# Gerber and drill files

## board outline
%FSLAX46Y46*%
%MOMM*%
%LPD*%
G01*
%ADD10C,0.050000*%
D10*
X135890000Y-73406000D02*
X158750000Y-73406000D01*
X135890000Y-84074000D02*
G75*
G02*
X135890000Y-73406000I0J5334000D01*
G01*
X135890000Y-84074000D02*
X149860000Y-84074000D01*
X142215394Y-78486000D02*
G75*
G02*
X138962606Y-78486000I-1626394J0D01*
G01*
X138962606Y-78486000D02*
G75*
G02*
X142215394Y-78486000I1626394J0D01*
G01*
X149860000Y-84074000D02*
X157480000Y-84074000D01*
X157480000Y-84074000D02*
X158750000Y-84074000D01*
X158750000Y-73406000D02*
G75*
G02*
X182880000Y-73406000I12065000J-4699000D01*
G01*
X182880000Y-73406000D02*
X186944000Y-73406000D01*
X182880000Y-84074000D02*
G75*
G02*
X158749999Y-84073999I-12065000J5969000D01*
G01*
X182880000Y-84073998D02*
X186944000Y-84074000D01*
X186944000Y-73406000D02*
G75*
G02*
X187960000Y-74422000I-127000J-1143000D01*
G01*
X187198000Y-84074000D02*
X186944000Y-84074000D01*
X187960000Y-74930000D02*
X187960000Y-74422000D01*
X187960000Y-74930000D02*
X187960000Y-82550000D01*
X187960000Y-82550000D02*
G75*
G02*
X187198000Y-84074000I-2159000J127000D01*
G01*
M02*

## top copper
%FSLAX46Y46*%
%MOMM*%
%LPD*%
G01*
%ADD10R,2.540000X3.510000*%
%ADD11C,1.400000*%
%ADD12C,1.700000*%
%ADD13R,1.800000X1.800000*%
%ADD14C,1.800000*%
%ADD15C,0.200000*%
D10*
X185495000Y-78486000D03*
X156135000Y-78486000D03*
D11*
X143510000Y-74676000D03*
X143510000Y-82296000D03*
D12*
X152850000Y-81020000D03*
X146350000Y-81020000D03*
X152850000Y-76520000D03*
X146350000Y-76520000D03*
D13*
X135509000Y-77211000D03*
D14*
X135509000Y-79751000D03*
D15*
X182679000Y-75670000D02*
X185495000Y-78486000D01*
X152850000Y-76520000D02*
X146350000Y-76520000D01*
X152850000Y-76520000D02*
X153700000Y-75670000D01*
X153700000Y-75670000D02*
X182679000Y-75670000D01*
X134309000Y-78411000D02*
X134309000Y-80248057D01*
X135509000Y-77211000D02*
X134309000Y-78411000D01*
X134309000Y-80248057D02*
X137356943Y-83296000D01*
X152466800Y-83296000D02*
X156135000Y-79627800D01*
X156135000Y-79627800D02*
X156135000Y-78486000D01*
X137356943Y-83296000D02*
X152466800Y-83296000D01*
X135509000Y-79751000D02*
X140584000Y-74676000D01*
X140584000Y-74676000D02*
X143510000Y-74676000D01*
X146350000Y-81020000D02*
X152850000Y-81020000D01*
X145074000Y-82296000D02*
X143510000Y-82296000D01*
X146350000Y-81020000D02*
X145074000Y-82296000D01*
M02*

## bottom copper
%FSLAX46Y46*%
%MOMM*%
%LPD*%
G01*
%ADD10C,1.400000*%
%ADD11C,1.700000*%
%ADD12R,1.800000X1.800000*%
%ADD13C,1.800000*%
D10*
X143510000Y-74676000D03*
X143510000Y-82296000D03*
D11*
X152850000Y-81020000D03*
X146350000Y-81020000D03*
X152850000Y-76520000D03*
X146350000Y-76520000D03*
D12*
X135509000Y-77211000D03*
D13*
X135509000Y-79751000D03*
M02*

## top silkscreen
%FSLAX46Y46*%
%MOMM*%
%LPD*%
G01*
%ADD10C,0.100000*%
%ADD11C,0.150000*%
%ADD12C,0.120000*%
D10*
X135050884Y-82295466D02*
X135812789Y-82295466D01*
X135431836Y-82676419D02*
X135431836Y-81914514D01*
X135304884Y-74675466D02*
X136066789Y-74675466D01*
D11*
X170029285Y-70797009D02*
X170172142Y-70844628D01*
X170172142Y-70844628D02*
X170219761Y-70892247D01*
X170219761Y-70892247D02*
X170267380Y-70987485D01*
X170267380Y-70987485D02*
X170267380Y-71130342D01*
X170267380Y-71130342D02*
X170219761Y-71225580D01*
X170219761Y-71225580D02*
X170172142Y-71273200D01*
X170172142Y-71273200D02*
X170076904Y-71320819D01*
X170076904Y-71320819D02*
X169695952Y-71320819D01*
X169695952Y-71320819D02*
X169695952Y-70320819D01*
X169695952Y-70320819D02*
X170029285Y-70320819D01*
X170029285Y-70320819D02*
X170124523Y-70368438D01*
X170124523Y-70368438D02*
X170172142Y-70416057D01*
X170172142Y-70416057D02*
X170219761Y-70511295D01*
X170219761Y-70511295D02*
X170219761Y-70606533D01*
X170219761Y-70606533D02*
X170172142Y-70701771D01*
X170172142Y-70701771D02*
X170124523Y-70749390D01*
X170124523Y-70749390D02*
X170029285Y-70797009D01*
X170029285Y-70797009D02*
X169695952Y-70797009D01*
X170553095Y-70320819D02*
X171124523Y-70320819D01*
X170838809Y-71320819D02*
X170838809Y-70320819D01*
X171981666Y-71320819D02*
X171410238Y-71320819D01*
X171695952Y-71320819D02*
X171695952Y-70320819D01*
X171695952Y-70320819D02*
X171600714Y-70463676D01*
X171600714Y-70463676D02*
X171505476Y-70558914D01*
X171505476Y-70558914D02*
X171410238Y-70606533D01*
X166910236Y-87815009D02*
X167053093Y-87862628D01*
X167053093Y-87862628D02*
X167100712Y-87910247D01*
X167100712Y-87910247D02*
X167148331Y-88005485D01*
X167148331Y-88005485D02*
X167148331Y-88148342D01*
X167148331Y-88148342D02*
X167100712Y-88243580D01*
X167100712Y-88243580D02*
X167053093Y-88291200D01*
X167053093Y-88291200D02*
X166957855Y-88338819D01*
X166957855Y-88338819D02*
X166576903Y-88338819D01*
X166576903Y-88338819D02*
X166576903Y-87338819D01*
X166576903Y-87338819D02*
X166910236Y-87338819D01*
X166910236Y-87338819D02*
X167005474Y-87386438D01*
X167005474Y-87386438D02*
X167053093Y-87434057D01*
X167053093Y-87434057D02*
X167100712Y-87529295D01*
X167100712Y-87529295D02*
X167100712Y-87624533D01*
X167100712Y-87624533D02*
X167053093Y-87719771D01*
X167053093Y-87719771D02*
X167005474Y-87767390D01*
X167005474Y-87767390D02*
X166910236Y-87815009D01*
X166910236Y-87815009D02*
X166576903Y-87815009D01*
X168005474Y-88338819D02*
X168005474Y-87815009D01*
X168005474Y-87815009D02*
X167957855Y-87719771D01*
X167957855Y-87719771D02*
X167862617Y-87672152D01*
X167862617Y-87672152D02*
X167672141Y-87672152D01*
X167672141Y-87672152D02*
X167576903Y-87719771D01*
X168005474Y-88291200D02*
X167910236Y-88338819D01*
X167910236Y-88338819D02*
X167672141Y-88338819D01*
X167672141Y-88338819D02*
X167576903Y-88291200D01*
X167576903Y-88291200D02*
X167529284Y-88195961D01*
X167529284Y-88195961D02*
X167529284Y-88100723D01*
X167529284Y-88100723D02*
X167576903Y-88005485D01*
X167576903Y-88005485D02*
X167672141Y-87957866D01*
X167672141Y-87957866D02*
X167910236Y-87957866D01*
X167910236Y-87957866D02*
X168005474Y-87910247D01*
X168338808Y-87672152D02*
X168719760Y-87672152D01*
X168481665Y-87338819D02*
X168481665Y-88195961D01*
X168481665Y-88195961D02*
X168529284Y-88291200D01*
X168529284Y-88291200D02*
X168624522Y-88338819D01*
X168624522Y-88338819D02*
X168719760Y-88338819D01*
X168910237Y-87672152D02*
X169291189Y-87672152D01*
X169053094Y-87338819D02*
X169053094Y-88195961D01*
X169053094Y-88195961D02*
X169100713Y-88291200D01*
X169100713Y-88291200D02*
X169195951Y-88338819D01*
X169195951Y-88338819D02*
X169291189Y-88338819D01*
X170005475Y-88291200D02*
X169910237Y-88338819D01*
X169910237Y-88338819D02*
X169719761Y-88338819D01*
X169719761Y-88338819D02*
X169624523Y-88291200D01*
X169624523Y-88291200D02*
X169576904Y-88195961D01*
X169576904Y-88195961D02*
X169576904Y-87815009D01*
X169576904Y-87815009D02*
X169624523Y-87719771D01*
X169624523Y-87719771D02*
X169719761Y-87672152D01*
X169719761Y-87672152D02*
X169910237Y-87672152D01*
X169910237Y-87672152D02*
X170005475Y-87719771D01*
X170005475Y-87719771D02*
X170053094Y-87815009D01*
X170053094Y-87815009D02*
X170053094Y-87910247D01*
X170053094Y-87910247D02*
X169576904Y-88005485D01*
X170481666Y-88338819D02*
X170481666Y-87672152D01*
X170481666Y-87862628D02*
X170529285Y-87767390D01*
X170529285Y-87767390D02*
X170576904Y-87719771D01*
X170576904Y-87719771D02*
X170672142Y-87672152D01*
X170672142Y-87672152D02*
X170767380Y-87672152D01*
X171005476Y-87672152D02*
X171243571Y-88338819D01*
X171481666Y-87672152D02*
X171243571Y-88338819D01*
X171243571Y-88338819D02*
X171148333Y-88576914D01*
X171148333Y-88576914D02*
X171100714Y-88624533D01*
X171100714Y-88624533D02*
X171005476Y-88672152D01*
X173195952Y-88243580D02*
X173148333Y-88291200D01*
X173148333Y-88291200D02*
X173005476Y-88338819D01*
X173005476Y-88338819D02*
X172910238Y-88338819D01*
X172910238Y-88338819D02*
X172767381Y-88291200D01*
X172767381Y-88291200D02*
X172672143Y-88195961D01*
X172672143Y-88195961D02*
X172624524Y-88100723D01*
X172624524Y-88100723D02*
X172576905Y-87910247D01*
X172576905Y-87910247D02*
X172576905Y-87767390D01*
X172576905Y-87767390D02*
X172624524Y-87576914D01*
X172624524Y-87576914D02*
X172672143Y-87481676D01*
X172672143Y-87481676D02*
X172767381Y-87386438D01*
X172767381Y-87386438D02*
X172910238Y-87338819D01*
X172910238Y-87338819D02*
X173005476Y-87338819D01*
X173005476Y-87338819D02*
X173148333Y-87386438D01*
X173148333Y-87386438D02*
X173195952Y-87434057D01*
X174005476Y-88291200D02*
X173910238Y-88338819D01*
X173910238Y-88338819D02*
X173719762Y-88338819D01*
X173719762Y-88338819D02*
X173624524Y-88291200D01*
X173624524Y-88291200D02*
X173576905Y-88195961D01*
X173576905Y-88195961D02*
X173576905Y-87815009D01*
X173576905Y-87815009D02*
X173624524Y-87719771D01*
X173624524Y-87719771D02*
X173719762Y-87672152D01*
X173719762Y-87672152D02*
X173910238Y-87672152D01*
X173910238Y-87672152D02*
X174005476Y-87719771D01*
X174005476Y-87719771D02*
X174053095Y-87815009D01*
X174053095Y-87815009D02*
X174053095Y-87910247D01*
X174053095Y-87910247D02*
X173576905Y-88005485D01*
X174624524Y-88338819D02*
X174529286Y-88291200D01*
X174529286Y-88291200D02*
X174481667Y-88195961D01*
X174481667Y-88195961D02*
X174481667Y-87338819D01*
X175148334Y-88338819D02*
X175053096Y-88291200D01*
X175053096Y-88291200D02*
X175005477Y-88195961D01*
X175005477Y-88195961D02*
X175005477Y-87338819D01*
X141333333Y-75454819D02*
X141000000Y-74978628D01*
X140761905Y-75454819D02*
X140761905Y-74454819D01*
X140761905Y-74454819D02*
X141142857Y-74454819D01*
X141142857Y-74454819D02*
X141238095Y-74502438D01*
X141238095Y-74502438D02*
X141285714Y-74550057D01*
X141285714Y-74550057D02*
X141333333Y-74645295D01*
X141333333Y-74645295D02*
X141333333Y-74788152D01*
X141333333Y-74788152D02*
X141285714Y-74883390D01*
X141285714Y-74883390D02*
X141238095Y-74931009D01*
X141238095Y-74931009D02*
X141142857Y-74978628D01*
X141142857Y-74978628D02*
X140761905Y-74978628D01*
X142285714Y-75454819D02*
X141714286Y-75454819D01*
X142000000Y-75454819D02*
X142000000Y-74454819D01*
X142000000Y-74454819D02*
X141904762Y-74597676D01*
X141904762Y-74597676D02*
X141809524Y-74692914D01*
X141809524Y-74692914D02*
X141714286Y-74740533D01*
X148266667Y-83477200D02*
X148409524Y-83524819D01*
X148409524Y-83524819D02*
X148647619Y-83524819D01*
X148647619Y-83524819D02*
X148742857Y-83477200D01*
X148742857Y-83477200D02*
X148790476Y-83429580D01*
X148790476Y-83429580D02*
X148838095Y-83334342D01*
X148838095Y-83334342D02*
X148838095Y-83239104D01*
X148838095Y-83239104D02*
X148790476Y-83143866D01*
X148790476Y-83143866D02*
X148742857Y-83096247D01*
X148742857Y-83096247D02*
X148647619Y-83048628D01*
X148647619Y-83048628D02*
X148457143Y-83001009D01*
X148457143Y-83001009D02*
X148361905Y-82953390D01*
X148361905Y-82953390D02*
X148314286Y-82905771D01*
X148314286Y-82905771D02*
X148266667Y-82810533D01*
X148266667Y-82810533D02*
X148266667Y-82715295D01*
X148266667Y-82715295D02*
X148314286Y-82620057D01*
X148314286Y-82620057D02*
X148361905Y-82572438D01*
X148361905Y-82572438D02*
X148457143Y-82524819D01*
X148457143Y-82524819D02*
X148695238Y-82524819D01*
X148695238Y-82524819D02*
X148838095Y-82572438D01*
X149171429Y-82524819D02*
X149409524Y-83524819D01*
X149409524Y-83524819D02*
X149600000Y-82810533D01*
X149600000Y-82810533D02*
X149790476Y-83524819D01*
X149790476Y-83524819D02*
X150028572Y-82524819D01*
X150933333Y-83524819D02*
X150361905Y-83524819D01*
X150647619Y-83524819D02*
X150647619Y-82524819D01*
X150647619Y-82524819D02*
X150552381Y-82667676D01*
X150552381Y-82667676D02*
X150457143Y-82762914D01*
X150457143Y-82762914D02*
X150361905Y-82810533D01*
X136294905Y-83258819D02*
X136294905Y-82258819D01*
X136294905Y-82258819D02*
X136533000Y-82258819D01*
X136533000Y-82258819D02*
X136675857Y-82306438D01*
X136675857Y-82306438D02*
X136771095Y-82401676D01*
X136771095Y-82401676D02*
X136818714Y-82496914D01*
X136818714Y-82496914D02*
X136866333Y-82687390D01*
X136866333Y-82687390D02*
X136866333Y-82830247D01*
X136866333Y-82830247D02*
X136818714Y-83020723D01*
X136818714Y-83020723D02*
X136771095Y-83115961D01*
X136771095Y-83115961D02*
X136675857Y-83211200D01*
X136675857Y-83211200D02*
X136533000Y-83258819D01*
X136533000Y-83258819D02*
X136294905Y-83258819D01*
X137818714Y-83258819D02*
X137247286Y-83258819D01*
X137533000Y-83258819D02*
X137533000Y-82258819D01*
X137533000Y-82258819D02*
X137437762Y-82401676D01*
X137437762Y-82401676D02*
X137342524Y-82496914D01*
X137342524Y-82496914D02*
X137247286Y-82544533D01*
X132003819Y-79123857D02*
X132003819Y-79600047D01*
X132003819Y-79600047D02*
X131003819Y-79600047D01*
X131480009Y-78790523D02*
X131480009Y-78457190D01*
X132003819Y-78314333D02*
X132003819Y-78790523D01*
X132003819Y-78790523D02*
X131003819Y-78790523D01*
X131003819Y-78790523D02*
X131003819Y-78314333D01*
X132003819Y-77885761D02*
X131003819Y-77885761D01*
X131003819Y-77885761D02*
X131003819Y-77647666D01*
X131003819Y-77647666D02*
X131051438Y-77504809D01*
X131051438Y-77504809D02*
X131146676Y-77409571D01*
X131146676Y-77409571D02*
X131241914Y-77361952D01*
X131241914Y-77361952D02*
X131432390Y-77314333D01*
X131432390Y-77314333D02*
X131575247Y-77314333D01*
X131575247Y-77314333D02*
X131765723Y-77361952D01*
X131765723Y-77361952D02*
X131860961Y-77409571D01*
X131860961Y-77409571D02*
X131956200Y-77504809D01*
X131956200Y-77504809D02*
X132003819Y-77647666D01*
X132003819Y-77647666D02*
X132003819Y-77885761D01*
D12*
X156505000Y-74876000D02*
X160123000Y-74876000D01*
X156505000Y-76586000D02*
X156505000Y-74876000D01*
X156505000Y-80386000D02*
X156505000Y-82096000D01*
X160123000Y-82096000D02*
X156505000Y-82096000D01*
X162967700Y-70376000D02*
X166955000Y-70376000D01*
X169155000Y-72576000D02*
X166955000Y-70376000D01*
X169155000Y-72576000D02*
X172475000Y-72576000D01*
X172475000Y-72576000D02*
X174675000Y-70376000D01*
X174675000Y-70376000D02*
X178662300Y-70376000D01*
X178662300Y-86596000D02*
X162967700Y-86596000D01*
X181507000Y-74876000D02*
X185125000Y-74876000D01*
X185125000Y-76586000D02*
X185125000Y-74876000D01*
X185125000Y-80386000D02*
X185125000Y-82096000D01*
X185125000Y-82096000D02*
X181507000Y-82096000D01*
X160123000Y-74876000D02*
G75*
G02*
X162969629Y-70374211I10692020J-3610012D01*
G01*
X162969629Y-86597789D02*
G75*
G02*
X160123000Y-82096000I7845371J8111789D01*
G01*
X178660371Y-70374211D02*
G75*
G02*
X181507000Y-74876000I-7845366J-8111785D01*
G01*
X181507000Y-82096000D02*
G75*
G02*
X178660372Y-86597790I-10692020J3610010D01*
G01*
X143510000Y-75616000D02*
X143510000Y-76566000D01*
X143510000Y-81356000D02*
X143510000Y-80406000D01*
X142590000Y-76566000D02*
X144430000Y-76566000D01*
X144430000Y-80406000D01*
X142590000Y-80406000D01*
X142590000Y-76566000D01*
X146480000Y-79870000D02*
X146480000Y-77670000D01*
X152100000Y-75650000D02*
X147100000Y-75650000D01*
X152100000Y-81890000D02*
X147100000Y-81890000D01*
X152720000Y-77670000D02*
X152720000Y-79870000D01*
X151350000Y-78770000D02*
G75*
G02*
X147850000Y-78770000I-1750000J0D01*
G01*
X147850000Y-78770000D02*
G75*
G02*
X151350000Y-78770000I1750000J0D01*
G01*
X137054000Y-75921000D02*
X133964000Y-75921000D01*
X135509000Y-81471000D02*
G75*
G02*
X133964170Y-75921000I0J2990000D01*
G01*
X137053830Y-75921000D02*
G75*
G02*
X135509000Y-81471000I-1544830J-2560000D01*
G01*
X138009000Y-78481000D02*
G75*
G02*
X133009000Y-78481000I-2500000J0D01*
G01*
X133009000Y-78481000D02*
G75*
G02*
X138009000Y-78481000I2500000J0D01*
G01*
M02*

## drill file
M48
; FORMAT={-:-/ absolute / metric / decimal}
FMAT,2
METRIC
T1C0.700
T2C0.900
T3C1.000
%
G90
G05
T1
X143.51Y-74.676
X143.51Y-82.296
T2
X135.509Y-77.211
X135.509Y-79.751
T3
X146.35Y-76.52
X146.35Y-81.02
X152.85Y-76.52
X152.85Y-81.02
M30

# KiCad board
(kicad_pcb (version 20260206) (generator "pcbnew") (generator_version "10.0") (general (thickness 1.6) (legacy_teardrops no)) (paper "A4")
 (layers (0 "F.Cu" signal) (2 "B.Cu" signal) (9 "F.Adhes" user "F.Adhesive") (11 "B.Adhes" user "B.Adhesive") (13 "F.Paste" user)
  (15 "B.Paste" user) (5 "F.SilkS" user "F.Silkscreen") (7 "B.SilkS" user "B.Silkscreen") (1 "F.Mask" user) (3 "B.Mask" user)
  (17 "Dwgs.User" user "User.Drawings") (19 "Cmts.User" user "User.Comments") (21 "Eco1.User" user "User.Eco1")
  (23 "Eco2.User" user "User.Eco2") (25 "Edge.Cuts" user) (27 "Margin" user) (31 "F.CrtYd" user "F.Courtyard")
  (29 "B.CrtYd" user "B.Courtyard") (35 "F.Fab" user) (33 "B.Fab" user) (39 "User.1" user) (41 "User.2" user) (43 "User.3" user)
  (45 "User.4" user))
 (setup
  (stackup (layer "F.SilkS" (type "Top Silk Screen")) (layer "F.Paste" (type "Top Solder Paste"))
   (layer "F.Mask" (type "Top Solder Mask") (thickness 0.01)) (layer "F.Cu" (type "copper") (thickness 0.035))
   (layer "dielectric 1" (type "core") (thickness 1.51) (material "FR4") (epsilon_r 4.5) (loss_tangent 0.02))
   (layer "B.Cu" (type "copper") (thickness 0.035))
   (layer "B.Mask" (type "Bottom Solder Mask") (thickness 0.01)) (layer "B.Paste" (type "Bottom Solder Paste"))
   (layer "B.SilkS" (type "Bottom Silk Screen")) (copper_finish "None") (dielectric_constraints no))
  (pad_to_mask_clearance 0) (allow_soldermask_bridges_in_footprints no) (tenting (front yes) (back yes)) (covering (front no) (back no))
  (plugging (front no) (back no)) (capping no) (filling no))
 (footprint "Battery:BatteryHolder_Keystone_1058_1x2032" (layer "F.Cu") (at 170.815 78.486 180)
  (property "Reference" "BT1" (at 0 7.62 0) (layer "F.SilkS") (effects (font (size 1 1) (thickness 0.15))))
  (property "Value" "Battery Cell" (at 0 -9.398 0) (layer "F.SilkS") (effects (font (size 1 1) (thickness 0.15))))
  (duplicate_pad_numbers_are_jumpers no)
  (fp_line (start 14.31 3.61) (end 10.692 3.61) (stroke (width 0.12) (type solid)) (layer "F.SilkS"))
  (fp_line (start 14.31 1.9) (end 14.31 3.61) (stroke (width 0.12) (type solid)) (layer "F.SilkS"))
  (fp_line (start 14.31 -1.9) (end 14.31 -3.61) (stroke (width 0.12) (type solid)) (layer "F.SilkS"))
  (fp_line (start 10.692 -3.61) (end 14.31 -3.61) (stroke (width 0.12) (type solid)) (layer "F.SilkS"))
  (fp_line (start 7.8473 8.11) (end 3.86 8.11) (stroke (width 0.12) (type solid)) (layer "F.SilkS"))
  (fp_line (start 1.66 5.91) (end 3.86 8.11) (stroke (width 0.12) (type solid)) (layer "F.SilkS"))
  (fp_line (start 1.66 5.91) (end -1.66 5.91) (stroke (width 0.12) (type solid)) (layer "F.SilkS"))
  (fp_line (start -1.66 5.91) (end -3.86 8.11) (stroke (width 0.12) (type solid)) (layer "F.SilkS"))
  (fp_line (start -3.86 8.11) (end -7.8473 8.11) (stroke (width 0.12) (type solid)) (layer "F.SilkS"))
  (fp_line (start -7.8473 -8.11) (end 7.8473 -8.11) (stroke (width 0.12) (type solid)) (layer "F.SilkS"))
  (fp_line (start -10.692 3.61) (end -14.31 3.61) (stroke (width 0.12) (type solid)) (layer "F.SilkS"))
  (fp_line (start -14.31 1.9) (end -14.31 3.61) (stroke (width 0.12) (type solid)) (layer "F.SilkS"))
  (fp_line (start -14.31 -1.9) (end -14.31 -3.61) (stroke (width 0.12) (type solid)) (layer "F.SilkS"))
  (fp_line (start -14.31 -3.61) (end -10.692 -3.61) (stroke (width 0.12) (type solid)) (layer "F.SilkS"))
  (fp_arc (start 10.692 3.61) (mid 9.538084 6.031244) (end 7.845371 8.111789) (stroke (width 0.12) (type solid)) (layer "F.SilkS"))
  (fp_arc (start 7.845371 -8.111789) (mid 9.538085 -6.031244) (end 10.692 -3.61) (stroke (width 0.12) (type solid)) (layer "F.SilkS"))
  (fp_arc (start -7.845371 8.111789) (mid -9.538085 6.031244) (end -10.692 3.61) (stroke (width 0.12) (type solid)) (layer "F.SilkS"))
  (fp_arc (start -10.692 -3.61) (mid -9.538084 -6.031244) (end -7.845371 -8.111789) (stroke (width 0.12) (type solid)) (layer "F.SilkS"))
  (pad "1" smd rect (at -14.68 0 180) (size 2.54 3.51) (layers "F.Cu" "F.Mask" "F.Paste") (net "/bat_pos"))
  (pad "2" smd rect (at 14.68 0 180) (size 2.54 3.51) (layers "F.Cu" "F.Mask" "F.Paste") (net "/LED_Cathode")))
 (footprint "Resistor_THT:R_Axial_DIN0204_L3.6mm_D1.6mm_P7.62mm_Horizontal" (layer "F.Cu") (at 143.51 74.676 -90)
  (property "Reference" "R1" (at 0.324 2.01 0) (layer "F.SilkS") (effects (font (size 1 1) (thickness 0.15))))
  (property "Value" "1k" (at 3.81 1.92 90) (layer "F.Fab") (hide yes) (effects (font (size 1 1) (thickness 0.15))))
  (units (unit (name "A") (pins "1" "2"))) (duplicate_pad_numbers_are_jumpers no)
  (fp_line (start 0.94 0) (end 1.89 0) (stroke (width 0.12) (type solid)) (layer "F.SilkS"))
  (fp_line (start 6.68 0) (end 5.73 0) (stroke (width 0.12) (type solid)) (layer "F.SilkS"))
  (fp_rect (start 1.89 -0.92) (end 5.73 0.92) (stroke (width 0.12) (type solid)) (fill no) (layer "F.SilkS"))
  (pad "1" thru_hole circle (at 0 0 270) (size 1.4 1.4) (drill 0.7) (layers "*.Cu" "*.Mask") (remove_unused_layers no) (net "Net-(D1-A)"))
  (pad "2" thru_hole circle (at 7.62 0 270) (size 1.4 1.4) (drill 0.7) (layers "*.Cu" "*.Mask") (remove_unused_layers no)
   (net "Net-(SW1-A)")))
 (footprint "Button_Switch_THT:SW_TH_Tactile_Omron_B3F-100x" (layer "F.Cu") (at 152.85 81.02 180)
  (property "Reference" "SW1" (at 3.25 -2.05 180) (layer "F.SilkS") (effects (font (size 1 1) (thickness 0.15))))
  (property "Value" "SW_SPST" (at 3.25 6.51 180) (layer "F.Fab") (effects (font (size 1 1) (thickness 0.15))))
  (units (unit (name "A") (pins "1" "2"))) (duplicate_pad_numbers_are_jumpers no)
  (fp_line (start 6.37 1.15) (end 6.37 3.35) (stroke (width 0.12) (type solid)) (layer "F.SilkS"))
  (fp_line (start 0.75 5.37) (end 5.75 5.37) (stroke (width 0.12) (type solid)) (layer "F.SilkS"))
  (fp_line (start 0.75 -0.87) (end 5.75 -0.87) (stroke (width 0.12) (type solid)) (layer "F.SilkS"))
  (fp_line (start 0.13 3.35) (end 0.13 1.15) (stroke (width 0.12) (type solid)) (layer "F.SilkS"))
  (fp_circle (center 3.25 2.25) (end 5 2.25) (stroke (width 0.12) (type solid)) (fill no) (layer "F.SilkS"))
  (pad "1" thru_hole circle (at 0 0 180) (size 1.7 1.7) (drill 1) (layers "*.Cu" "*.Mask") (remove_unused_layers no) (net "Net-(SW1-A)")
   (thermal_bridge_angle 90))
  (pad "1" thru_hole circle (at 6.5 0 180) (size 1.7 1.7) (drill 1) (layers "*.Cu" "*.Mask") (remove_unused_layers no) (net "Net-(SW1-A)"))
  (pad "2" thru_hole circle (at 0 4.5 180) (size 1.7 1.7) (drill 1) (layers "*.Cu" "*.Mask") (remove_unused_layers no) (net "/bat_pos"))
  (pad "2" thru_hole circle (at 6.5 4.5 180) (size 1.7 1.7) (drill 1) (layers "*.Cu" "*.Mask") (remove_unused_layers no) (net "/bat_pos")))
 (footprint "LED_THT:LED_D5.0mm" (layer "F.Cu") (at 135.509 77.211 -90)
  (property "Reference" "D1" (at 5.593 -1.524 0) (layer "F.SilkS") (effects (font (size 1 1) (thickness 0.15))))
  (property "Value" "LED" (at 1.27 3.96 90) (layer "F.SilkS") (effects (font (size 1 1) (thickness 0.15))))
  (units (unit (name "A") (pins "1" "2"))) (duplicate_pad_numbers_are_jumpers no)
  (fp_line (start -1.29 -1.545) (end -1.29 1.545) (stroke (width 0.12) (type solid)) (layer "F.SilkS"))
  (fp_arc (start 4.26 0) (mid 2.071779 2.880495) (end -1.29 1.54483) (stroke (width 0.12) (type solid)) (layer "F.SilkS"))
  (fp_arc (start -1.29 -1.54483) (mid 2.071779 -2.880495) (end 4.26 0) (stroke (width 0.12) (type solid)) (layer "F.SilkS"))
  (fp_circle (center 1.27 0) (end 3.77 0) (stroke (width 0.12) (type solid)) (fill no) (layer "F.SilkS"))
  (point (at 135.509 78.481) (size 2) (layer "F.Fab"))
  (pad "1" thru_hole rect (at 0 0 270) (size 1.8 1.8) (drill 0.9) (layers "*.Cu" "*.Mask") (remove_unused_layers no) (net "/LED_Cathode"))
  (pad "2" thru_hole circle (at 2.54 0 270) (size 1.8 1.8) (drill 0.9) (layers "*.Cu" "*.Mask") (remove_unused_layers no) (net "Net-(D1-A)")))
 (gr_line (start 135.89 73.406) (end 158.75 73.406) (stroke (width 0.05) (type default)) (locked yes) (layer "Edge.Cuts"))
 (gr_arc (start 135.89 84.074) (mid 130.556 78.74) (end 135.89 73.406) (stroke (width 0.05) (type default)) (locked yes) (layer "Edge.Cuts"))
 (gr_line (start 135.89 84.074) (end 149.86 84.074) (stroke (width 0.05) (type default)) (locked yes) (layer "Edge.Cuts"))
 (gr_circle (center 140.589 78.486) (end 141.605 79.756) (stroke (width 0.05) (type default)) (fill no) (layer "Edge.Cuts"))
 (gr_line (start 149.86 84.074) (end 157.48 84.074) (stroke (width 0.05) (type default)) (locked yes) (layer "Edge.Cuts"))
 (gr_line (start 157.48 84.074) (end 158.75 84.074) (stroke (width 0.05) (type default)) (locked yes) (layer "Edge.Cuts"))
 (gr_arc (start 158.75 73.406) (mid 170.815 65.157227) (end 182.88 73.406) (stroke (width 0.05) (type default)) (locked yes)
  (layer "Edge.Cuts"))
 (gr_line (start 182.88 73.406) (end 186.944 73.406) (stroke (width 0.05) (type default)) (locked yes) (layer "Edge.Cuts"))
 (gr_arc (start 182.88 84.074) (mid 170.814999 91.565802) (end 158.749999 84.073999) (stroke (width 0.05) (type default)) (locked yes)
  (layer "Edge.Cuts"))
 (gr_line (start 182.88 84.073998) (end 186.944 84.074) (stroke (width 0.05) (type default)) (locked yes) (layer "Edge.Cuts"))
 (gr_arc (start 186.944 73.406) (mid 187.630197 73.735803) (end 187.96 74.422) (stroke (width 0.05) (type default)) (locked yes)
  (layer "Edge.Cuts"))
 (gr_line (start 187.198 84.074) (end 186.944 84.074) (stroke (width 0.05) (type default)) (locked yes) (layer "Edge.Cuts"))
 (gr_line (start 187.96 74.93) (end 187.96 74.422) (stroke (width 0.05) (type default)) (locked yes) (layer "Edge.Cuts"))
 (gr_line (start 187.96 74.93) (end 187.96 82.55) (stroke (width 0.05) (type default)) (locked yes) (layer "Edge.Cuts"))
 (gr_arc (start 187.96 82.55) (mid 187.735406 83.390203) (end 187.198 84.074) (stroke (width 0.05) (type default)) (locked yes)
  (layer "Edge.Cuts"))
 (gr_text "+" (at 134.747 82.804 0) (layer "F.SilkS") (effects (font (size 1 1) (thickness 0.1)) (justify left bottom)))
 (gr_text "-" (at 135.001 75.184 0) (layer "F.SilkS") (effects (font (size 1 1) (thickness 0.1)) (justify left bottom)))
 (segment (start 182.679 75.67) (end 185.495 78.486) (width 0.2) (layer "F.Cu") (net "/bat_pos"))
 (segment (start 152.85 76.52) (end 146.35 76.52) (width 0.2) (layer "F.Cu") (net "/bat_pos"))
 (segment (start 152.85 76.52) (end 153.7 75.67) (width 0.2) (layer "F.Cu") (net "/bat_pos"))
 (segment (start 153.7 75.67) (end 182.679 75.67) (width 0.2) (layer "F.Cu") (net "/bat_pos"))
 (segment (start 134.309 78.411) (end 134.309 80.248057) (width 0.2) (layer "F.Cu") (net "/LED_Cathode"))
 (segment (start 135.509 77.211) (end 134.309 78.411) (width 0.2) (layer "F.Cu") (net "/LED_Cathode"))
 (segment (start 134.309 80.248057) (end 137.356943 83.296) (width 0.2) (layer "F.Cu") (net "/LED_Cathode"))
 (segment (start 152.4668 83.296) (end 156.135 79.6278) (width 0.2) (layer "F.Cu") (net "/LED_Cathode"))
 (segment (start 156.135 79.6278) (end 156.135 78.486) (width 0.2) (layer "F.Cu") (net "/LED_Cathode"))
 (segment (start 137.356943 83.296) (end 152.4668 83.296) (width 0.2) (layer "F.Cu") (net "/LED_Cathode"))
 (segment (start 135.509 79.751) (end 140.584 74.676) (width 0.2) (layer "F.Cu") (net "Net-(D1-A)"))
 (segment (start 140.584 74.676) (end 143.51 74.676) (width 0.2) (layer "F.Cu") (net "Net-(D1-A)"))
 (segment (start 146.35 81.02) (end 152.85 81.02) (width 0.2) (layer "F.Cu") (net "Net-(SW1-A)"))
 (segment (start 145.074 82.296) (end 143.51 82.296) (width 0.2) (layer "F.Cu") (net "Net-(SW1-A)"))
 (segment (start 146.35 81.02) (end 145.074 82.296) (width 0.2) (layer "F.Cu") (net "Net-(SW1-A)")))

